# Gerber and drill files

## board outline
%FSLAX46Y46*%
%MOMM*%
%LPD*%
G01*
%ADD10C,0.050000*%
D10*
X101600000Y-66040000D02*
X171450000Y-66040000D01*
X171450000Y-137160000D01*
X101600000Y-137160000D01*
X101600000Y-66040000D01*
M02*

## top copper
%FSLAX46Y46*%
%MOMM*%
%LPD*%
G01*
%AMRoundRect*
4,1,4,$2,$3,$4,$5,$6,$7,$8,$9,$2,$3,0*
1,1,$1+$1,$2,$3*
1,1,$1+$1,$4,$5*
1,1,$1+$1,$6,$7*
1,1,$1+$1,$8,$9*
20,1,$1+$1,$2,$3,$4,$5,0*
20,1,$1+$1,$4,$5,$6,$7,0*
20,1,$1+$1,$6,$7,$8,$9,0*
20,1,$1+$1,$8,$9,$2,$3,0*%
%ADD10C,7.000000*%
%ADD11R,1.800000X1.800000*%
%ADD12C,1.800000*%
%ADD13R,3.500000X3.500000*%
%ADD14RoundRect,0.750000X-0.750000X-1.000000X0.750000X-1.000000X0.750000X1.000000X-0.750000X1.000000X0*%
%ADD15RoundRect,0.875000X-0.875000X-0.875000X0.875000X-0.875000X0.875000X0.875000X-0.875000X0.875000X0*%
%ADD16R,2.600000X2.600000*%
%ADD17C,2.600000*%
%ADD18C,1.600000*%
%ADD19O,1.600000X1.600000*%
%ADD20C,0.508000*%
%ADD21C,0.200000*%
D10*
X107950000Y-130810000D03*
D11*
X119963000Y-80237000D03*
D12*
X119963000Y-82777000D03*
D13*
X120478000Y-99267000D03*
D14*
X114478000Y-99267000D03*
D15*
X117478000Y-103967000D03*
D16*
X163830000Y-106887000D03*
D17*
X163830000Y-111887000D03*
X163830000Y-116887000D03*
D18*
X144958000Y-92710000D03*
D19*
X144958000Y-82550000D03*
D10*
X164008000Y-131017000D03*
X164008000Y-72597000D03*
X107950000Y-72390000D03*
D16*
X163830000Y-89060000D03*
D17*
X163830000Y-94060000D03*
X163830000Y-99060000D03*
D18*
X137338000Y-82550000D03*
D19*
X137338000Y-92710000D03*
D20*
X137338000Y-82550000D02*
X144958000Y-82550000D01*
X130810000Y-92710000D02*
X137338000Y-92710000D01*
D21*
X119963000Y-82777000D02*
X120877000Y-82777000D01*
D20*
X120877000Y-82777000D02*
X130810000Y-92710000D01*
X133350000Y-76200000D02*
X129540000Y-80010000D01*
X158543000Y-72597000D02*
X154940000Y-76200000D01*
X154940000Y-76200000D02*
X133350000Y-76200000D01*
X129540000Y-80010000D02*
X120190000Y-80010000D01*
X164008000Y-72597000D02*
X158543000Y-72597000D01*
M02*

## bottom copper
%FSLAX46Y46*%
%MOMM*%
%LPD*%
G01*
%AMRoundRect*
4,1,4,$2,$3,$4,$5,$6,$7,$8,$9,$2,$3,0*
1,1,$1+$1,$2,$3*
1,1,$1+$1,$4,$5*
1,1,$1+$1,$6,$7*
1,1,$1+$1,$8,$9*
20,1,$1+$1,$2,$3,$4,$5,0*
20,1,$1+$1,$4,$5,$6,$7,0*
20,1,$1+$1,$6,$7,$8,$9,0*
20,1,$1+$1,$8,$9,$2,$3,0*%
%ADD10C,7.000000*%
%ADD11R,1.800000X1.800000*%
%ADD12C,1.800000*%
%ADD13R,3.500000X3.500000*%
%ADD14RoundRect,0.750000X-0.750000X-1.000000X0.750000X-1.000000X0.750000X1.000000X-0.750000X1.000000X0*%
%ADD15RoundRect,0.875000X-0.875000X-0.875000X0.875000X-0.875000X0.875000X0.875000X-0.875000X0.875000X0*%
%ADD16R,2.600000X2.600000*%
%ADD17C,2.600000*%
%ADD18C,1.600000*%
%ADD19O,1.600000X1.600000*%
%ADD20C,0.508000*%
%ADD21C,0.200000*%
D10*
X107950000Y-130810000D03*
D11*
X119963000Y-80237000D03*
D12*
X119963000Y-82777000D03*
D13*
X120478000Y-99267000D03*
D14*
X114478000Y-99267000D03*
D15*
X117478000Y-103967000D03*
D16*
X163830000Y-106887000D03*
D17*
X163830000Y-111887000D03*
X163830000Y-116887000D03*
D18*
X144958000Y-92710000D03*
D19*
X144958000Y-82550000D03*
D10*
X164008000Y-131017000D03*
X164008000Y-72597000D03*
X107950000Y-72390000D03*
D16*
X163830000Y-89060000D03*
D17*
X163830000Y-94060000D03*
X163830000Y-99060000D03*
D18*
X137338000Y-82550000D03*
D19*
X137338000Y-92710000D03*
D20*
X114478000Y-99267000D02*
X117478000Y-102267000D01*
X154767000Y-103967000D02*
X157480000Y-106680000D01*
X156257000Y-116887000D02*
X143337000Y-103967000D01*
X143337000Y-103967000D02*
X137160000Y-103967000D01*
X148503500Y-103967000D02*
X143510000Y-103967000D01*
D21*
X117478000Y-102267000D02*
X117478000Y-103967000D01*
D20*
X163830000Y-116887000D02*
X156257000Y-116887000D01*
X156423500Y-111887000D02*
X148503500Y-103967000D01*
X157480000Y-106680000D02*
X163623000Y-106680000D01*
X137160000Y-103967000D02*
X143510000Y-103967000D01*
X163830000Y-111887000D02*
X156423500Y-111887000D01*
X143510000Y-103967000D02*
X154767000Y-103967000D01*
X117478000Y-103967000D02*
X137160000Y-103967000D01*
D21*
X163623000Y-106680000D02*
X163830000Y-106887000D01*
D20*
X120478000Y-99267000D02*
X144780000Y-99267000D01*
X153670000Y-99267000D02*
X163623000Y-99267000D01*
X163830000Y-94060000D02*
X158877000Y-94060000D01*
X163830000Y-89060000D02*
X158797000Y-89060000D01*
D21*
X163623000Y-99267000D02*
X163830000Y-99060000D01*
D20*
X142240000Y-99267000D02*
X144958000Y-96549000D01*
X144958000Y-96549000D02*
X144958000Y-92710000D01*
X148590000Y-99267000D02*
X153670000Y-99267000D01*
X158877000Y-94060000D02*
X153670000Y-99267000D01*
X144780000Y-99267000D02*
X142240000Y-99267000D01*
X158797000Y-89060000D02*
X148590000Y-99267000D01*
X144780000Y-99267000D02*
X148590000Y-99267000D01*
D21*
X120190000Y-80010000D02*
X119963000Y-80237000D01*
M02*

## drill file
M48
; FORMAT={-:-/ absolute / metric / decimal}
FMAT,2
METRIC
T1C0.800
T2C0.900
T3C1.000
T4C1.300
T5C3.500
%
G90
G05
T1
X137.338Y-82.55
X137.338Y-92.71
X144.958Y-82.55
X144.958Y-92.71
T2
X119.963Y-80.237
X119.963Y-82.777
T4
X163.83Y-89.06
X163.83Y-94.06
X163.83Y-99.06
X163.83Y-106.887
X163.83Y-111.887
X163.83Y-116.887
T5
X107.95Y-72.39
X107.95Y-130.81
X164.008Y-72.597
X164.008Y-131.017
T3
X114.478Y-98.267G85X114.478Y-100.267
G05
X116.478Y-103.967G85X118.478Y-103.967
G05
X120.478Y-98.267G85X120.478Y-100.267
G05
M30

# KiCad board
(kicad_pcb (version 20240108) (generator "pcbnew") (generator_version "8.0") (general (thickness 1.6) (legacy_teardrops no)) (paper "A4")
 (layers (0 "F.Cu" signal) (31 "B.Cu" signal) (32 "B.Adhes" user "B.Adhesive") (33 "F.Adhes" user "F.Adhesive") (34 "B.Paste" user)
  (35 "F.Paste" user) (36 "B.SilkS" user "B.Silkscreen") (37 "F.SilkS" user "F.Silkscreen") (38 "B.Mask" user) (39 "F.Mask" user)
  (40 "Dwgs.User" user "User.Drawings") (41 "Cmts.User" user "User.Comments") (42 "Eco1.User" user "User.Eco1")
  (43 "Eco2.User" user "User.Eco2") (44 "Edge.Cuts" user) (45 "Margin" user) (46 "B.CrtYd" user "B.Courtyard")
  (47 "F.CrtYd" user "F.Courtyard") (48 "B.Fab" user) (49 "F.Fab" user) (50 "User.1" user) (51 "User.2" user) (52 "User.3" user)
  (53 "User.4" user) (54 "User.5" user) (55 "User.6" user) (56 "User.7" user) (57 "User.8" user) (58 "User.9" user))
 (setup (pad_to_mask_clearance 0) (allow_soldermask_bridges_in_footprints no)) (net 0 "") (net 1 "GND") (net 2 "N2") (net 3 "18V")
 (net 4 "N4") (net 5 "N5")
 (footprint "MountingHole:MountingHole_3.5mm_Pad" (layer "F.Cu") (at 107.95 130.81)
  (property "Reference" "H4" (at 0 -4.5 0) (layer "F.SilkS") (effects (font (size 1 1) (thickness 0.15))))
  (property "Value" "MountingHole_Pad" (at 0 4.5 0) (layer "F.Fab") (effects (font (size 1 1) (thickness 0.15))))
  (pad "1" thru_hole circle (at 0 0) (size 7 7) (drill 3.5) (layers "*.Cu" "*.Mask") (remove_unused_layers no) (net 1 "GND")))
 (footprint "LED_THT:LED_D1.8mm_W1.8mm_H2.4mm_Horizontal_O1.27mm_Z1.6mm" (layer "F.Cu") (at 119.963 80.237 -90)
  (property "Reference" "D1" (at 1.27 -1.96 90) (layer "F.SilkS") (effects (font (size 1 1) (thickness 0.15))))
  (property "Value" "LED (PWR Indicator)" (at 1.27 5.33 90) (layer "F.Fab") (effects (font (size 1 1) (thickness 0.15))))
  (pad "1" thru_hole rect (at 0 0 270) (size 1.8 1.8) (drill 0.9) (layers "*.Cu" "*.Mask") (remove_unused_layers no) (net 1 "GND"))
  (pad "2" thru_hole circle (at 2.54 0 270) (size 1.8 1.8) (drill 0.9) (layers "*.Cu" "*.Mask") (remove_unused_layers no) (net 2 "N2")))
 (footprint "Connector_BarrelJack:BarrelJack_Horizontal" (layer "F.Cu") (at 120.478 99.267)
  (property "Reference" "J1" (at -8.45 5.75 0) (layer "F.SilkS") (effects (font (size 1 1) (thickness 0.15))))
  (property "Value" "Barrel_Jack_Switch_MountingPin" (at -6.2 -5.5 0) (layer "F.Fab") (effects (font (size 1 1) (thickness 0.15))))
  (pad "1" thru_hole rect (at 0 0) (size 3.5 3.5) (drill oval 1 3) (layers "*.Cu" "*.Mask") (remove_unused_layers no) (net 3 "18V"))
  (pad "2" thru_hole roundrect (at -6 0) (size 3 3.5) (drill oval 1 3) (layers "*.Cu" "*.Mask") (remove_unused_layers no)
   (roundrect_rratio 0.25) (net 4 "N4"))
  (pad "3" thru_hole roundrect (at -3 4.7) (size 3.5 3.5) (drill oval 3 1) (layers "*.Cu" "*.Mask") (remove_unused_layers no)
   (roundrect_rratio 0.25) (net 4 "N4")))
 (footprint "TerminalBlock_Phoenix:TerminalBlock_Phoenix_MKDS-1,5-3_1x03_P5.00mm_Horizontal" (layer "F.Cu") (at 163.83 106.887 -90)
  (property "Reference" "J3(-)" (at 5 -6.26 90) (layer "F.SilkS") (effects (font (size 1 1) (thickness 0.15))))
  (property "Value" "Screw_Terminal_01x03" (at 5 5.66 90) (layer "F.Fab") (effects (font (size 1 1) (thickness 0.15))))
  (pad "1" thru_hole rect (at 0 0 270) (size 2.6 2.6) (drill 1.3) (layers "*.Cu" "*.Mask") (remove_unused_layers no) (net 4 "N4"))
  (pad "2" thru_hole circle (at 5 0 270) (size 2.6 2.6) (drill 1.3) (layers "*.Cu" "*.Mask") (remove_unused_layers no) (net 4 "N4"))
  (pad "3" thru_hole circle (at 10 0 270) (size 2.6 2.6) (drill 1.3) (layers "*.Cu" "*.Mask") (remove_unused_layers no) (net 4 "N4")))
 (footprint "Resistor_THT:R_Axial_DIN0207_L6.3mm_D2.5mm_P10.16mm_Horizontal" (layer "F.Cu") (at 144.958 92.71 90)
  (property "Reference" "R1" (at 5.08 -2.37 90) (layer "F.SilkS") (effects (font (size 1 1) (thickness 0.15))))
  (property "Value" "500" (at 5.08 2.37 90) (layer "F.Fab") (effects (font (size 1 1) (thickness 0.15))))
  (pad "1" thru_hole circle (at 0 0 90) (size 1.6 1.6) (drill 0.8) (layers "*.Cu" "*.Mask") (remove_unused_layers no) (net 3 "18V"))
  (pad "2" thru_hole oval (at 10.16 0 90) (size 1.6 1.6) (drill 0.8) (layers "*.Cu" "*.Mask") (remove_unused_layers no) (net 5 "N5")))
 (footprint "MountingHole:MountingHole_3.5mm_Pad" (layer "F.Cu") (at 164.008 131.017)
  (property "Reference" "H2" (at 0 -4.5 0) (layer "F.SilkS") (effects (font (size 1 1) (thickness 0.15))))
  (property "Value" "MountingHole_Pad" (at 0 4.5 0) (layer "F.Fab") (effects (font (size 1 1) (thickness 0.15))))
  (pad "1" thru_hole circle (at 0 0) (size 7 7) (drill 3.5) (layers "*.Cu" "*.Mask") (remove_unused_layers no) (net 1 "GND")))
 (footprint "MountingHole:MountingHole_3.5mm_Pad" (layer "F.Cu") (at 164.008 72.597)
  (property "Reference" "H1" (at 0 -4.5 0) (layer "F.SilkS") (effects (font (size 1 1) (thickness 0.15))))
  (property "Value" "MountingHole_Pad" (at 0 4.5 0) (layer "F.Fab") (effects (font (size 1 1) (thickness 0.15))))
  (pad "1" thru_hole circle (at 0 0) (size 7 7) (drill 3.5) (layers "*.Cu" "*.Mask") (remove_unused_layers no) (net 1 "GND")))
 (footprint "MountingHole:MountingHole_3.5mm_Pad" (layer "F.Cu") (at 107.95 72.39)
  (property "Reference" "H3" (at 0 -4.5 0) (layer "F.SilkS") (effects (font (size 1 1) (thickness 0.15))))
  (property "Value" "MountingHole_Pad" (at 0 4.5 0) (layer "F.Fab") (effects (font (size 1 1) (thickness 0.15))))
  (pad "1" thru_hole circle (at 0 0) (size 7 7) (drill 3.5) (layers "*.Cu" "*.Mask") (remove_unused_layers no) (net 1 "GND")))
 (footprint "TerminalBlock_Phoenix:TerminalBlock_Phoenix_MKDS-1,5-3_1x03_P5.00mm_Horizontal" (layer "F.Cu") (at 163.83 89.06 -90)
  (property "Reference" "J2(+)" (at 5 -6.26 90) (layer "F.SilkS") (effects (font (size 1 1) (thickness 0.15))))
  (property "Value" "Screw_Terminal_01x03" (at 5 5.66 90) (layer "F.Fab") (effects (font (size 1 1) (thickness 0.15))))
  (pad "1" thru_hole rect (at 0 0 270) (size 2.6 2.6) (drill 1.3) (layers "*.Cu" "*.Mask") (remove_unused_layers no) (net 3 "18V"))
  (pad "2" thru_hole circle (at 5 0 270) (size 2.6 2.6) (drill 1.3) (layers "*.Cu" "*.Mask") (remove_unused_layers no) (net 3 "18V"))
  (pad "3" thru_hole circle (at 10 0 270) (size 2.6 2.6) (drill 1.3) (layers "*.Cu" "*.Mask") (remove_unused_layers no) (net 3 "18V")))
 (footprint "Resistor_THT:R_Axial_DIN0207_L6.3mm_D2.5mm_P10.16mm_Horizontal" (layer "F.Cu") (at 137.338 82.55 -90)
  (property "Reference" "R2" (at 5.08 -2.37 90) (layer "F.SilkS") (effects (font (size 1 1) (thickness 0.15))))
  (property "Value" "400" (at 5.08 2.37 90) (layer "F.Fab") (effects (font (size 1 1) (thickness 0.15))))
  (pad "1" thru_hole circle (at 0 0 270) (size 1.6 1.6) (drill 0.8) (layers "*.Cu" "*.Mask") (remove_unused_layers no) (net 5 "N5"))
  (pad "2" thru_hole oval (at 10.16 0 270) (size 1.6 1.6) (drill 0.8) (layers "*.Cu" "*.Mask") (remove_unused_layers no) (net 2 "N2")))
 (gr_rect (start 101.6 66.04) (end 171.45 137.16) (stroke (width 0.05) (type default)) (fill none) (layer "Edge.Cuts"))
 (segment (start 114.478 99.267) (end 117.478 102.267) (width 0.508) (layer "B.Cu") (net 4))
 (segment (start 154.767 103.967) (end 157.48 106.68) (width 0.508) (layer "B.Cu") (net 4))
 (segment (start 156.257 116.887) (end 143.337 103.967) (width 0.508) (layer "B.Cu") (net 4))
 (segment (start 143.337 103.967) (end 137.16 103.967) (width 0.508) (layer "B.Cu") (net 4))
 (segment (start 148.5035 103.967) (end 143.51 103.967) (width 0.508) (layer "B.Cu") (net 4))
 (segment (start 117.478 102.267) (end 117.478 103.967) (width 0.2) (layer "B.Cu") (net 4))
 (segment (start 163.83 116.887) (end 156.257 116.887) (width 0.508) (layer "B.Cu") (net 4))
 (segment (start 156.4235 111.887) (end 148.5035 103.967) (width 0.508) (layer "B.Cu") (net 4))
 (segment (start 157.48 106.68) (end 163.623 106.68) (width 0.508) (layer "B.Cu") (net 4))
 (segment (start 137.16 103.967) (end 143.51 103.967) (width 0.508) (layer "B.Cu") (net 4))
 (segment (start 163.83 111.887) (end 156.4235 111.887) (width 0.508) (layer "B.Cu") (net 4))
 (segment (start 143.51 103.967) (end 154.767 103.967) (width 0.508) (layer "B.Cu") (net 4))
 (segment (start 117.478 103.967) (end 137.16 103.967) (width 0.508) (layer "B.Cu") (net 4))
 (segment (start 163.623 106.68) (end 163.83 106.887) (width 0.2) (layer "B.Cu") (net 4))
 (segment (start 137.338 82.55) (end 144.958 82.55) (width 0.508) (layer "F.Cu") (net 5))
 (segment (start 120.478 99.267) (end 144.78 99.267) (width 0.508) (layer "B.Cu") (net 3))
 (segment (start 153.67 99.267) (end 163.623 99.267) (width 0.508) (layer "B.Cu") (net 3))
 (segment (start 163.83 94.06) (end 158.877 94.06) (width 0.508) (layer "B.Cu") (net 3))
 (segment (start 163.83 89.06) (end 158.797 89.06) (width 0.508) (layer "B.Cu") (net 3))
 (segment (start 163.623 99.267) (end 163.83 99.06) (width 0.2) (layer "B.Cu") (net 3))
 (segment (start 142.24 99.267) (end 144.958 96.549) (width 0.508) (layer "B.Cu") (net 3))
 (segment (start 144.958 96.549) (end 144.958 92.71) (width 0.508) (layer "B.Cu") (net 3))
 (segment (start 148.59 99.267) (end 153.67 99.267) (width 0.508) (layer "B.Cu") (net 3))
 (segment (start 158.877 94.06) (end 153.67 99.267) (width 0.508) (layer "B.Cu") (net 3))
 (segment (start 144.78 99.267) (end 142.24 99.267) (width 0.508) (layer "B.Cu") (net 3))
 (segment (start 158.797 89.06) (end 148.59 99.267) (width 0.508) (layer "B.Cu") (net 3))
 (segment (start 144.78 99.267) (end 148.59 99.267) (width 0.508) (layer "B.Cu") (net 3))
 (segment (start 130.81 92.71) (end 137.338 92.71) (width 0.508) (layer "F.Cu") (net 2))
 (segment (start 119.963 82.777) (end 120.877 82.777) (width 0.2) (layer "F.Cu") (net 2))
 (segment (start 120.877 82.777) (end 130.81 92.71) (width 0.508) (layer "F.Cu") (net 2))
 (segment (start 133.35 76.2) (end 129.54 80.01) (width 0.508) (layer "F.Cu") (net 1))
 (segment (start 158.543 72.597) (end 154.94 76.2) (width 0.508) (layer "F.Cu") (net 1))
 (segment (start 154.94 76.2) (end 133.35 76.2) (width 0.508) (layer "F.Cu") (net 1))
 (segment (start 129.54 80.01) (end 120.19 80.01) (width 0.508) (layer "F.Cu") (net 1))
 (segment (start 164.008 72.597) (end 158.543 72.597) (width 0.508) (layer "F.Cu") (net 1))
 (segment (start 120.19 80.01) (end 119.963 80.237) (width 0.2) (layer "B.Cu") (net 1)))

